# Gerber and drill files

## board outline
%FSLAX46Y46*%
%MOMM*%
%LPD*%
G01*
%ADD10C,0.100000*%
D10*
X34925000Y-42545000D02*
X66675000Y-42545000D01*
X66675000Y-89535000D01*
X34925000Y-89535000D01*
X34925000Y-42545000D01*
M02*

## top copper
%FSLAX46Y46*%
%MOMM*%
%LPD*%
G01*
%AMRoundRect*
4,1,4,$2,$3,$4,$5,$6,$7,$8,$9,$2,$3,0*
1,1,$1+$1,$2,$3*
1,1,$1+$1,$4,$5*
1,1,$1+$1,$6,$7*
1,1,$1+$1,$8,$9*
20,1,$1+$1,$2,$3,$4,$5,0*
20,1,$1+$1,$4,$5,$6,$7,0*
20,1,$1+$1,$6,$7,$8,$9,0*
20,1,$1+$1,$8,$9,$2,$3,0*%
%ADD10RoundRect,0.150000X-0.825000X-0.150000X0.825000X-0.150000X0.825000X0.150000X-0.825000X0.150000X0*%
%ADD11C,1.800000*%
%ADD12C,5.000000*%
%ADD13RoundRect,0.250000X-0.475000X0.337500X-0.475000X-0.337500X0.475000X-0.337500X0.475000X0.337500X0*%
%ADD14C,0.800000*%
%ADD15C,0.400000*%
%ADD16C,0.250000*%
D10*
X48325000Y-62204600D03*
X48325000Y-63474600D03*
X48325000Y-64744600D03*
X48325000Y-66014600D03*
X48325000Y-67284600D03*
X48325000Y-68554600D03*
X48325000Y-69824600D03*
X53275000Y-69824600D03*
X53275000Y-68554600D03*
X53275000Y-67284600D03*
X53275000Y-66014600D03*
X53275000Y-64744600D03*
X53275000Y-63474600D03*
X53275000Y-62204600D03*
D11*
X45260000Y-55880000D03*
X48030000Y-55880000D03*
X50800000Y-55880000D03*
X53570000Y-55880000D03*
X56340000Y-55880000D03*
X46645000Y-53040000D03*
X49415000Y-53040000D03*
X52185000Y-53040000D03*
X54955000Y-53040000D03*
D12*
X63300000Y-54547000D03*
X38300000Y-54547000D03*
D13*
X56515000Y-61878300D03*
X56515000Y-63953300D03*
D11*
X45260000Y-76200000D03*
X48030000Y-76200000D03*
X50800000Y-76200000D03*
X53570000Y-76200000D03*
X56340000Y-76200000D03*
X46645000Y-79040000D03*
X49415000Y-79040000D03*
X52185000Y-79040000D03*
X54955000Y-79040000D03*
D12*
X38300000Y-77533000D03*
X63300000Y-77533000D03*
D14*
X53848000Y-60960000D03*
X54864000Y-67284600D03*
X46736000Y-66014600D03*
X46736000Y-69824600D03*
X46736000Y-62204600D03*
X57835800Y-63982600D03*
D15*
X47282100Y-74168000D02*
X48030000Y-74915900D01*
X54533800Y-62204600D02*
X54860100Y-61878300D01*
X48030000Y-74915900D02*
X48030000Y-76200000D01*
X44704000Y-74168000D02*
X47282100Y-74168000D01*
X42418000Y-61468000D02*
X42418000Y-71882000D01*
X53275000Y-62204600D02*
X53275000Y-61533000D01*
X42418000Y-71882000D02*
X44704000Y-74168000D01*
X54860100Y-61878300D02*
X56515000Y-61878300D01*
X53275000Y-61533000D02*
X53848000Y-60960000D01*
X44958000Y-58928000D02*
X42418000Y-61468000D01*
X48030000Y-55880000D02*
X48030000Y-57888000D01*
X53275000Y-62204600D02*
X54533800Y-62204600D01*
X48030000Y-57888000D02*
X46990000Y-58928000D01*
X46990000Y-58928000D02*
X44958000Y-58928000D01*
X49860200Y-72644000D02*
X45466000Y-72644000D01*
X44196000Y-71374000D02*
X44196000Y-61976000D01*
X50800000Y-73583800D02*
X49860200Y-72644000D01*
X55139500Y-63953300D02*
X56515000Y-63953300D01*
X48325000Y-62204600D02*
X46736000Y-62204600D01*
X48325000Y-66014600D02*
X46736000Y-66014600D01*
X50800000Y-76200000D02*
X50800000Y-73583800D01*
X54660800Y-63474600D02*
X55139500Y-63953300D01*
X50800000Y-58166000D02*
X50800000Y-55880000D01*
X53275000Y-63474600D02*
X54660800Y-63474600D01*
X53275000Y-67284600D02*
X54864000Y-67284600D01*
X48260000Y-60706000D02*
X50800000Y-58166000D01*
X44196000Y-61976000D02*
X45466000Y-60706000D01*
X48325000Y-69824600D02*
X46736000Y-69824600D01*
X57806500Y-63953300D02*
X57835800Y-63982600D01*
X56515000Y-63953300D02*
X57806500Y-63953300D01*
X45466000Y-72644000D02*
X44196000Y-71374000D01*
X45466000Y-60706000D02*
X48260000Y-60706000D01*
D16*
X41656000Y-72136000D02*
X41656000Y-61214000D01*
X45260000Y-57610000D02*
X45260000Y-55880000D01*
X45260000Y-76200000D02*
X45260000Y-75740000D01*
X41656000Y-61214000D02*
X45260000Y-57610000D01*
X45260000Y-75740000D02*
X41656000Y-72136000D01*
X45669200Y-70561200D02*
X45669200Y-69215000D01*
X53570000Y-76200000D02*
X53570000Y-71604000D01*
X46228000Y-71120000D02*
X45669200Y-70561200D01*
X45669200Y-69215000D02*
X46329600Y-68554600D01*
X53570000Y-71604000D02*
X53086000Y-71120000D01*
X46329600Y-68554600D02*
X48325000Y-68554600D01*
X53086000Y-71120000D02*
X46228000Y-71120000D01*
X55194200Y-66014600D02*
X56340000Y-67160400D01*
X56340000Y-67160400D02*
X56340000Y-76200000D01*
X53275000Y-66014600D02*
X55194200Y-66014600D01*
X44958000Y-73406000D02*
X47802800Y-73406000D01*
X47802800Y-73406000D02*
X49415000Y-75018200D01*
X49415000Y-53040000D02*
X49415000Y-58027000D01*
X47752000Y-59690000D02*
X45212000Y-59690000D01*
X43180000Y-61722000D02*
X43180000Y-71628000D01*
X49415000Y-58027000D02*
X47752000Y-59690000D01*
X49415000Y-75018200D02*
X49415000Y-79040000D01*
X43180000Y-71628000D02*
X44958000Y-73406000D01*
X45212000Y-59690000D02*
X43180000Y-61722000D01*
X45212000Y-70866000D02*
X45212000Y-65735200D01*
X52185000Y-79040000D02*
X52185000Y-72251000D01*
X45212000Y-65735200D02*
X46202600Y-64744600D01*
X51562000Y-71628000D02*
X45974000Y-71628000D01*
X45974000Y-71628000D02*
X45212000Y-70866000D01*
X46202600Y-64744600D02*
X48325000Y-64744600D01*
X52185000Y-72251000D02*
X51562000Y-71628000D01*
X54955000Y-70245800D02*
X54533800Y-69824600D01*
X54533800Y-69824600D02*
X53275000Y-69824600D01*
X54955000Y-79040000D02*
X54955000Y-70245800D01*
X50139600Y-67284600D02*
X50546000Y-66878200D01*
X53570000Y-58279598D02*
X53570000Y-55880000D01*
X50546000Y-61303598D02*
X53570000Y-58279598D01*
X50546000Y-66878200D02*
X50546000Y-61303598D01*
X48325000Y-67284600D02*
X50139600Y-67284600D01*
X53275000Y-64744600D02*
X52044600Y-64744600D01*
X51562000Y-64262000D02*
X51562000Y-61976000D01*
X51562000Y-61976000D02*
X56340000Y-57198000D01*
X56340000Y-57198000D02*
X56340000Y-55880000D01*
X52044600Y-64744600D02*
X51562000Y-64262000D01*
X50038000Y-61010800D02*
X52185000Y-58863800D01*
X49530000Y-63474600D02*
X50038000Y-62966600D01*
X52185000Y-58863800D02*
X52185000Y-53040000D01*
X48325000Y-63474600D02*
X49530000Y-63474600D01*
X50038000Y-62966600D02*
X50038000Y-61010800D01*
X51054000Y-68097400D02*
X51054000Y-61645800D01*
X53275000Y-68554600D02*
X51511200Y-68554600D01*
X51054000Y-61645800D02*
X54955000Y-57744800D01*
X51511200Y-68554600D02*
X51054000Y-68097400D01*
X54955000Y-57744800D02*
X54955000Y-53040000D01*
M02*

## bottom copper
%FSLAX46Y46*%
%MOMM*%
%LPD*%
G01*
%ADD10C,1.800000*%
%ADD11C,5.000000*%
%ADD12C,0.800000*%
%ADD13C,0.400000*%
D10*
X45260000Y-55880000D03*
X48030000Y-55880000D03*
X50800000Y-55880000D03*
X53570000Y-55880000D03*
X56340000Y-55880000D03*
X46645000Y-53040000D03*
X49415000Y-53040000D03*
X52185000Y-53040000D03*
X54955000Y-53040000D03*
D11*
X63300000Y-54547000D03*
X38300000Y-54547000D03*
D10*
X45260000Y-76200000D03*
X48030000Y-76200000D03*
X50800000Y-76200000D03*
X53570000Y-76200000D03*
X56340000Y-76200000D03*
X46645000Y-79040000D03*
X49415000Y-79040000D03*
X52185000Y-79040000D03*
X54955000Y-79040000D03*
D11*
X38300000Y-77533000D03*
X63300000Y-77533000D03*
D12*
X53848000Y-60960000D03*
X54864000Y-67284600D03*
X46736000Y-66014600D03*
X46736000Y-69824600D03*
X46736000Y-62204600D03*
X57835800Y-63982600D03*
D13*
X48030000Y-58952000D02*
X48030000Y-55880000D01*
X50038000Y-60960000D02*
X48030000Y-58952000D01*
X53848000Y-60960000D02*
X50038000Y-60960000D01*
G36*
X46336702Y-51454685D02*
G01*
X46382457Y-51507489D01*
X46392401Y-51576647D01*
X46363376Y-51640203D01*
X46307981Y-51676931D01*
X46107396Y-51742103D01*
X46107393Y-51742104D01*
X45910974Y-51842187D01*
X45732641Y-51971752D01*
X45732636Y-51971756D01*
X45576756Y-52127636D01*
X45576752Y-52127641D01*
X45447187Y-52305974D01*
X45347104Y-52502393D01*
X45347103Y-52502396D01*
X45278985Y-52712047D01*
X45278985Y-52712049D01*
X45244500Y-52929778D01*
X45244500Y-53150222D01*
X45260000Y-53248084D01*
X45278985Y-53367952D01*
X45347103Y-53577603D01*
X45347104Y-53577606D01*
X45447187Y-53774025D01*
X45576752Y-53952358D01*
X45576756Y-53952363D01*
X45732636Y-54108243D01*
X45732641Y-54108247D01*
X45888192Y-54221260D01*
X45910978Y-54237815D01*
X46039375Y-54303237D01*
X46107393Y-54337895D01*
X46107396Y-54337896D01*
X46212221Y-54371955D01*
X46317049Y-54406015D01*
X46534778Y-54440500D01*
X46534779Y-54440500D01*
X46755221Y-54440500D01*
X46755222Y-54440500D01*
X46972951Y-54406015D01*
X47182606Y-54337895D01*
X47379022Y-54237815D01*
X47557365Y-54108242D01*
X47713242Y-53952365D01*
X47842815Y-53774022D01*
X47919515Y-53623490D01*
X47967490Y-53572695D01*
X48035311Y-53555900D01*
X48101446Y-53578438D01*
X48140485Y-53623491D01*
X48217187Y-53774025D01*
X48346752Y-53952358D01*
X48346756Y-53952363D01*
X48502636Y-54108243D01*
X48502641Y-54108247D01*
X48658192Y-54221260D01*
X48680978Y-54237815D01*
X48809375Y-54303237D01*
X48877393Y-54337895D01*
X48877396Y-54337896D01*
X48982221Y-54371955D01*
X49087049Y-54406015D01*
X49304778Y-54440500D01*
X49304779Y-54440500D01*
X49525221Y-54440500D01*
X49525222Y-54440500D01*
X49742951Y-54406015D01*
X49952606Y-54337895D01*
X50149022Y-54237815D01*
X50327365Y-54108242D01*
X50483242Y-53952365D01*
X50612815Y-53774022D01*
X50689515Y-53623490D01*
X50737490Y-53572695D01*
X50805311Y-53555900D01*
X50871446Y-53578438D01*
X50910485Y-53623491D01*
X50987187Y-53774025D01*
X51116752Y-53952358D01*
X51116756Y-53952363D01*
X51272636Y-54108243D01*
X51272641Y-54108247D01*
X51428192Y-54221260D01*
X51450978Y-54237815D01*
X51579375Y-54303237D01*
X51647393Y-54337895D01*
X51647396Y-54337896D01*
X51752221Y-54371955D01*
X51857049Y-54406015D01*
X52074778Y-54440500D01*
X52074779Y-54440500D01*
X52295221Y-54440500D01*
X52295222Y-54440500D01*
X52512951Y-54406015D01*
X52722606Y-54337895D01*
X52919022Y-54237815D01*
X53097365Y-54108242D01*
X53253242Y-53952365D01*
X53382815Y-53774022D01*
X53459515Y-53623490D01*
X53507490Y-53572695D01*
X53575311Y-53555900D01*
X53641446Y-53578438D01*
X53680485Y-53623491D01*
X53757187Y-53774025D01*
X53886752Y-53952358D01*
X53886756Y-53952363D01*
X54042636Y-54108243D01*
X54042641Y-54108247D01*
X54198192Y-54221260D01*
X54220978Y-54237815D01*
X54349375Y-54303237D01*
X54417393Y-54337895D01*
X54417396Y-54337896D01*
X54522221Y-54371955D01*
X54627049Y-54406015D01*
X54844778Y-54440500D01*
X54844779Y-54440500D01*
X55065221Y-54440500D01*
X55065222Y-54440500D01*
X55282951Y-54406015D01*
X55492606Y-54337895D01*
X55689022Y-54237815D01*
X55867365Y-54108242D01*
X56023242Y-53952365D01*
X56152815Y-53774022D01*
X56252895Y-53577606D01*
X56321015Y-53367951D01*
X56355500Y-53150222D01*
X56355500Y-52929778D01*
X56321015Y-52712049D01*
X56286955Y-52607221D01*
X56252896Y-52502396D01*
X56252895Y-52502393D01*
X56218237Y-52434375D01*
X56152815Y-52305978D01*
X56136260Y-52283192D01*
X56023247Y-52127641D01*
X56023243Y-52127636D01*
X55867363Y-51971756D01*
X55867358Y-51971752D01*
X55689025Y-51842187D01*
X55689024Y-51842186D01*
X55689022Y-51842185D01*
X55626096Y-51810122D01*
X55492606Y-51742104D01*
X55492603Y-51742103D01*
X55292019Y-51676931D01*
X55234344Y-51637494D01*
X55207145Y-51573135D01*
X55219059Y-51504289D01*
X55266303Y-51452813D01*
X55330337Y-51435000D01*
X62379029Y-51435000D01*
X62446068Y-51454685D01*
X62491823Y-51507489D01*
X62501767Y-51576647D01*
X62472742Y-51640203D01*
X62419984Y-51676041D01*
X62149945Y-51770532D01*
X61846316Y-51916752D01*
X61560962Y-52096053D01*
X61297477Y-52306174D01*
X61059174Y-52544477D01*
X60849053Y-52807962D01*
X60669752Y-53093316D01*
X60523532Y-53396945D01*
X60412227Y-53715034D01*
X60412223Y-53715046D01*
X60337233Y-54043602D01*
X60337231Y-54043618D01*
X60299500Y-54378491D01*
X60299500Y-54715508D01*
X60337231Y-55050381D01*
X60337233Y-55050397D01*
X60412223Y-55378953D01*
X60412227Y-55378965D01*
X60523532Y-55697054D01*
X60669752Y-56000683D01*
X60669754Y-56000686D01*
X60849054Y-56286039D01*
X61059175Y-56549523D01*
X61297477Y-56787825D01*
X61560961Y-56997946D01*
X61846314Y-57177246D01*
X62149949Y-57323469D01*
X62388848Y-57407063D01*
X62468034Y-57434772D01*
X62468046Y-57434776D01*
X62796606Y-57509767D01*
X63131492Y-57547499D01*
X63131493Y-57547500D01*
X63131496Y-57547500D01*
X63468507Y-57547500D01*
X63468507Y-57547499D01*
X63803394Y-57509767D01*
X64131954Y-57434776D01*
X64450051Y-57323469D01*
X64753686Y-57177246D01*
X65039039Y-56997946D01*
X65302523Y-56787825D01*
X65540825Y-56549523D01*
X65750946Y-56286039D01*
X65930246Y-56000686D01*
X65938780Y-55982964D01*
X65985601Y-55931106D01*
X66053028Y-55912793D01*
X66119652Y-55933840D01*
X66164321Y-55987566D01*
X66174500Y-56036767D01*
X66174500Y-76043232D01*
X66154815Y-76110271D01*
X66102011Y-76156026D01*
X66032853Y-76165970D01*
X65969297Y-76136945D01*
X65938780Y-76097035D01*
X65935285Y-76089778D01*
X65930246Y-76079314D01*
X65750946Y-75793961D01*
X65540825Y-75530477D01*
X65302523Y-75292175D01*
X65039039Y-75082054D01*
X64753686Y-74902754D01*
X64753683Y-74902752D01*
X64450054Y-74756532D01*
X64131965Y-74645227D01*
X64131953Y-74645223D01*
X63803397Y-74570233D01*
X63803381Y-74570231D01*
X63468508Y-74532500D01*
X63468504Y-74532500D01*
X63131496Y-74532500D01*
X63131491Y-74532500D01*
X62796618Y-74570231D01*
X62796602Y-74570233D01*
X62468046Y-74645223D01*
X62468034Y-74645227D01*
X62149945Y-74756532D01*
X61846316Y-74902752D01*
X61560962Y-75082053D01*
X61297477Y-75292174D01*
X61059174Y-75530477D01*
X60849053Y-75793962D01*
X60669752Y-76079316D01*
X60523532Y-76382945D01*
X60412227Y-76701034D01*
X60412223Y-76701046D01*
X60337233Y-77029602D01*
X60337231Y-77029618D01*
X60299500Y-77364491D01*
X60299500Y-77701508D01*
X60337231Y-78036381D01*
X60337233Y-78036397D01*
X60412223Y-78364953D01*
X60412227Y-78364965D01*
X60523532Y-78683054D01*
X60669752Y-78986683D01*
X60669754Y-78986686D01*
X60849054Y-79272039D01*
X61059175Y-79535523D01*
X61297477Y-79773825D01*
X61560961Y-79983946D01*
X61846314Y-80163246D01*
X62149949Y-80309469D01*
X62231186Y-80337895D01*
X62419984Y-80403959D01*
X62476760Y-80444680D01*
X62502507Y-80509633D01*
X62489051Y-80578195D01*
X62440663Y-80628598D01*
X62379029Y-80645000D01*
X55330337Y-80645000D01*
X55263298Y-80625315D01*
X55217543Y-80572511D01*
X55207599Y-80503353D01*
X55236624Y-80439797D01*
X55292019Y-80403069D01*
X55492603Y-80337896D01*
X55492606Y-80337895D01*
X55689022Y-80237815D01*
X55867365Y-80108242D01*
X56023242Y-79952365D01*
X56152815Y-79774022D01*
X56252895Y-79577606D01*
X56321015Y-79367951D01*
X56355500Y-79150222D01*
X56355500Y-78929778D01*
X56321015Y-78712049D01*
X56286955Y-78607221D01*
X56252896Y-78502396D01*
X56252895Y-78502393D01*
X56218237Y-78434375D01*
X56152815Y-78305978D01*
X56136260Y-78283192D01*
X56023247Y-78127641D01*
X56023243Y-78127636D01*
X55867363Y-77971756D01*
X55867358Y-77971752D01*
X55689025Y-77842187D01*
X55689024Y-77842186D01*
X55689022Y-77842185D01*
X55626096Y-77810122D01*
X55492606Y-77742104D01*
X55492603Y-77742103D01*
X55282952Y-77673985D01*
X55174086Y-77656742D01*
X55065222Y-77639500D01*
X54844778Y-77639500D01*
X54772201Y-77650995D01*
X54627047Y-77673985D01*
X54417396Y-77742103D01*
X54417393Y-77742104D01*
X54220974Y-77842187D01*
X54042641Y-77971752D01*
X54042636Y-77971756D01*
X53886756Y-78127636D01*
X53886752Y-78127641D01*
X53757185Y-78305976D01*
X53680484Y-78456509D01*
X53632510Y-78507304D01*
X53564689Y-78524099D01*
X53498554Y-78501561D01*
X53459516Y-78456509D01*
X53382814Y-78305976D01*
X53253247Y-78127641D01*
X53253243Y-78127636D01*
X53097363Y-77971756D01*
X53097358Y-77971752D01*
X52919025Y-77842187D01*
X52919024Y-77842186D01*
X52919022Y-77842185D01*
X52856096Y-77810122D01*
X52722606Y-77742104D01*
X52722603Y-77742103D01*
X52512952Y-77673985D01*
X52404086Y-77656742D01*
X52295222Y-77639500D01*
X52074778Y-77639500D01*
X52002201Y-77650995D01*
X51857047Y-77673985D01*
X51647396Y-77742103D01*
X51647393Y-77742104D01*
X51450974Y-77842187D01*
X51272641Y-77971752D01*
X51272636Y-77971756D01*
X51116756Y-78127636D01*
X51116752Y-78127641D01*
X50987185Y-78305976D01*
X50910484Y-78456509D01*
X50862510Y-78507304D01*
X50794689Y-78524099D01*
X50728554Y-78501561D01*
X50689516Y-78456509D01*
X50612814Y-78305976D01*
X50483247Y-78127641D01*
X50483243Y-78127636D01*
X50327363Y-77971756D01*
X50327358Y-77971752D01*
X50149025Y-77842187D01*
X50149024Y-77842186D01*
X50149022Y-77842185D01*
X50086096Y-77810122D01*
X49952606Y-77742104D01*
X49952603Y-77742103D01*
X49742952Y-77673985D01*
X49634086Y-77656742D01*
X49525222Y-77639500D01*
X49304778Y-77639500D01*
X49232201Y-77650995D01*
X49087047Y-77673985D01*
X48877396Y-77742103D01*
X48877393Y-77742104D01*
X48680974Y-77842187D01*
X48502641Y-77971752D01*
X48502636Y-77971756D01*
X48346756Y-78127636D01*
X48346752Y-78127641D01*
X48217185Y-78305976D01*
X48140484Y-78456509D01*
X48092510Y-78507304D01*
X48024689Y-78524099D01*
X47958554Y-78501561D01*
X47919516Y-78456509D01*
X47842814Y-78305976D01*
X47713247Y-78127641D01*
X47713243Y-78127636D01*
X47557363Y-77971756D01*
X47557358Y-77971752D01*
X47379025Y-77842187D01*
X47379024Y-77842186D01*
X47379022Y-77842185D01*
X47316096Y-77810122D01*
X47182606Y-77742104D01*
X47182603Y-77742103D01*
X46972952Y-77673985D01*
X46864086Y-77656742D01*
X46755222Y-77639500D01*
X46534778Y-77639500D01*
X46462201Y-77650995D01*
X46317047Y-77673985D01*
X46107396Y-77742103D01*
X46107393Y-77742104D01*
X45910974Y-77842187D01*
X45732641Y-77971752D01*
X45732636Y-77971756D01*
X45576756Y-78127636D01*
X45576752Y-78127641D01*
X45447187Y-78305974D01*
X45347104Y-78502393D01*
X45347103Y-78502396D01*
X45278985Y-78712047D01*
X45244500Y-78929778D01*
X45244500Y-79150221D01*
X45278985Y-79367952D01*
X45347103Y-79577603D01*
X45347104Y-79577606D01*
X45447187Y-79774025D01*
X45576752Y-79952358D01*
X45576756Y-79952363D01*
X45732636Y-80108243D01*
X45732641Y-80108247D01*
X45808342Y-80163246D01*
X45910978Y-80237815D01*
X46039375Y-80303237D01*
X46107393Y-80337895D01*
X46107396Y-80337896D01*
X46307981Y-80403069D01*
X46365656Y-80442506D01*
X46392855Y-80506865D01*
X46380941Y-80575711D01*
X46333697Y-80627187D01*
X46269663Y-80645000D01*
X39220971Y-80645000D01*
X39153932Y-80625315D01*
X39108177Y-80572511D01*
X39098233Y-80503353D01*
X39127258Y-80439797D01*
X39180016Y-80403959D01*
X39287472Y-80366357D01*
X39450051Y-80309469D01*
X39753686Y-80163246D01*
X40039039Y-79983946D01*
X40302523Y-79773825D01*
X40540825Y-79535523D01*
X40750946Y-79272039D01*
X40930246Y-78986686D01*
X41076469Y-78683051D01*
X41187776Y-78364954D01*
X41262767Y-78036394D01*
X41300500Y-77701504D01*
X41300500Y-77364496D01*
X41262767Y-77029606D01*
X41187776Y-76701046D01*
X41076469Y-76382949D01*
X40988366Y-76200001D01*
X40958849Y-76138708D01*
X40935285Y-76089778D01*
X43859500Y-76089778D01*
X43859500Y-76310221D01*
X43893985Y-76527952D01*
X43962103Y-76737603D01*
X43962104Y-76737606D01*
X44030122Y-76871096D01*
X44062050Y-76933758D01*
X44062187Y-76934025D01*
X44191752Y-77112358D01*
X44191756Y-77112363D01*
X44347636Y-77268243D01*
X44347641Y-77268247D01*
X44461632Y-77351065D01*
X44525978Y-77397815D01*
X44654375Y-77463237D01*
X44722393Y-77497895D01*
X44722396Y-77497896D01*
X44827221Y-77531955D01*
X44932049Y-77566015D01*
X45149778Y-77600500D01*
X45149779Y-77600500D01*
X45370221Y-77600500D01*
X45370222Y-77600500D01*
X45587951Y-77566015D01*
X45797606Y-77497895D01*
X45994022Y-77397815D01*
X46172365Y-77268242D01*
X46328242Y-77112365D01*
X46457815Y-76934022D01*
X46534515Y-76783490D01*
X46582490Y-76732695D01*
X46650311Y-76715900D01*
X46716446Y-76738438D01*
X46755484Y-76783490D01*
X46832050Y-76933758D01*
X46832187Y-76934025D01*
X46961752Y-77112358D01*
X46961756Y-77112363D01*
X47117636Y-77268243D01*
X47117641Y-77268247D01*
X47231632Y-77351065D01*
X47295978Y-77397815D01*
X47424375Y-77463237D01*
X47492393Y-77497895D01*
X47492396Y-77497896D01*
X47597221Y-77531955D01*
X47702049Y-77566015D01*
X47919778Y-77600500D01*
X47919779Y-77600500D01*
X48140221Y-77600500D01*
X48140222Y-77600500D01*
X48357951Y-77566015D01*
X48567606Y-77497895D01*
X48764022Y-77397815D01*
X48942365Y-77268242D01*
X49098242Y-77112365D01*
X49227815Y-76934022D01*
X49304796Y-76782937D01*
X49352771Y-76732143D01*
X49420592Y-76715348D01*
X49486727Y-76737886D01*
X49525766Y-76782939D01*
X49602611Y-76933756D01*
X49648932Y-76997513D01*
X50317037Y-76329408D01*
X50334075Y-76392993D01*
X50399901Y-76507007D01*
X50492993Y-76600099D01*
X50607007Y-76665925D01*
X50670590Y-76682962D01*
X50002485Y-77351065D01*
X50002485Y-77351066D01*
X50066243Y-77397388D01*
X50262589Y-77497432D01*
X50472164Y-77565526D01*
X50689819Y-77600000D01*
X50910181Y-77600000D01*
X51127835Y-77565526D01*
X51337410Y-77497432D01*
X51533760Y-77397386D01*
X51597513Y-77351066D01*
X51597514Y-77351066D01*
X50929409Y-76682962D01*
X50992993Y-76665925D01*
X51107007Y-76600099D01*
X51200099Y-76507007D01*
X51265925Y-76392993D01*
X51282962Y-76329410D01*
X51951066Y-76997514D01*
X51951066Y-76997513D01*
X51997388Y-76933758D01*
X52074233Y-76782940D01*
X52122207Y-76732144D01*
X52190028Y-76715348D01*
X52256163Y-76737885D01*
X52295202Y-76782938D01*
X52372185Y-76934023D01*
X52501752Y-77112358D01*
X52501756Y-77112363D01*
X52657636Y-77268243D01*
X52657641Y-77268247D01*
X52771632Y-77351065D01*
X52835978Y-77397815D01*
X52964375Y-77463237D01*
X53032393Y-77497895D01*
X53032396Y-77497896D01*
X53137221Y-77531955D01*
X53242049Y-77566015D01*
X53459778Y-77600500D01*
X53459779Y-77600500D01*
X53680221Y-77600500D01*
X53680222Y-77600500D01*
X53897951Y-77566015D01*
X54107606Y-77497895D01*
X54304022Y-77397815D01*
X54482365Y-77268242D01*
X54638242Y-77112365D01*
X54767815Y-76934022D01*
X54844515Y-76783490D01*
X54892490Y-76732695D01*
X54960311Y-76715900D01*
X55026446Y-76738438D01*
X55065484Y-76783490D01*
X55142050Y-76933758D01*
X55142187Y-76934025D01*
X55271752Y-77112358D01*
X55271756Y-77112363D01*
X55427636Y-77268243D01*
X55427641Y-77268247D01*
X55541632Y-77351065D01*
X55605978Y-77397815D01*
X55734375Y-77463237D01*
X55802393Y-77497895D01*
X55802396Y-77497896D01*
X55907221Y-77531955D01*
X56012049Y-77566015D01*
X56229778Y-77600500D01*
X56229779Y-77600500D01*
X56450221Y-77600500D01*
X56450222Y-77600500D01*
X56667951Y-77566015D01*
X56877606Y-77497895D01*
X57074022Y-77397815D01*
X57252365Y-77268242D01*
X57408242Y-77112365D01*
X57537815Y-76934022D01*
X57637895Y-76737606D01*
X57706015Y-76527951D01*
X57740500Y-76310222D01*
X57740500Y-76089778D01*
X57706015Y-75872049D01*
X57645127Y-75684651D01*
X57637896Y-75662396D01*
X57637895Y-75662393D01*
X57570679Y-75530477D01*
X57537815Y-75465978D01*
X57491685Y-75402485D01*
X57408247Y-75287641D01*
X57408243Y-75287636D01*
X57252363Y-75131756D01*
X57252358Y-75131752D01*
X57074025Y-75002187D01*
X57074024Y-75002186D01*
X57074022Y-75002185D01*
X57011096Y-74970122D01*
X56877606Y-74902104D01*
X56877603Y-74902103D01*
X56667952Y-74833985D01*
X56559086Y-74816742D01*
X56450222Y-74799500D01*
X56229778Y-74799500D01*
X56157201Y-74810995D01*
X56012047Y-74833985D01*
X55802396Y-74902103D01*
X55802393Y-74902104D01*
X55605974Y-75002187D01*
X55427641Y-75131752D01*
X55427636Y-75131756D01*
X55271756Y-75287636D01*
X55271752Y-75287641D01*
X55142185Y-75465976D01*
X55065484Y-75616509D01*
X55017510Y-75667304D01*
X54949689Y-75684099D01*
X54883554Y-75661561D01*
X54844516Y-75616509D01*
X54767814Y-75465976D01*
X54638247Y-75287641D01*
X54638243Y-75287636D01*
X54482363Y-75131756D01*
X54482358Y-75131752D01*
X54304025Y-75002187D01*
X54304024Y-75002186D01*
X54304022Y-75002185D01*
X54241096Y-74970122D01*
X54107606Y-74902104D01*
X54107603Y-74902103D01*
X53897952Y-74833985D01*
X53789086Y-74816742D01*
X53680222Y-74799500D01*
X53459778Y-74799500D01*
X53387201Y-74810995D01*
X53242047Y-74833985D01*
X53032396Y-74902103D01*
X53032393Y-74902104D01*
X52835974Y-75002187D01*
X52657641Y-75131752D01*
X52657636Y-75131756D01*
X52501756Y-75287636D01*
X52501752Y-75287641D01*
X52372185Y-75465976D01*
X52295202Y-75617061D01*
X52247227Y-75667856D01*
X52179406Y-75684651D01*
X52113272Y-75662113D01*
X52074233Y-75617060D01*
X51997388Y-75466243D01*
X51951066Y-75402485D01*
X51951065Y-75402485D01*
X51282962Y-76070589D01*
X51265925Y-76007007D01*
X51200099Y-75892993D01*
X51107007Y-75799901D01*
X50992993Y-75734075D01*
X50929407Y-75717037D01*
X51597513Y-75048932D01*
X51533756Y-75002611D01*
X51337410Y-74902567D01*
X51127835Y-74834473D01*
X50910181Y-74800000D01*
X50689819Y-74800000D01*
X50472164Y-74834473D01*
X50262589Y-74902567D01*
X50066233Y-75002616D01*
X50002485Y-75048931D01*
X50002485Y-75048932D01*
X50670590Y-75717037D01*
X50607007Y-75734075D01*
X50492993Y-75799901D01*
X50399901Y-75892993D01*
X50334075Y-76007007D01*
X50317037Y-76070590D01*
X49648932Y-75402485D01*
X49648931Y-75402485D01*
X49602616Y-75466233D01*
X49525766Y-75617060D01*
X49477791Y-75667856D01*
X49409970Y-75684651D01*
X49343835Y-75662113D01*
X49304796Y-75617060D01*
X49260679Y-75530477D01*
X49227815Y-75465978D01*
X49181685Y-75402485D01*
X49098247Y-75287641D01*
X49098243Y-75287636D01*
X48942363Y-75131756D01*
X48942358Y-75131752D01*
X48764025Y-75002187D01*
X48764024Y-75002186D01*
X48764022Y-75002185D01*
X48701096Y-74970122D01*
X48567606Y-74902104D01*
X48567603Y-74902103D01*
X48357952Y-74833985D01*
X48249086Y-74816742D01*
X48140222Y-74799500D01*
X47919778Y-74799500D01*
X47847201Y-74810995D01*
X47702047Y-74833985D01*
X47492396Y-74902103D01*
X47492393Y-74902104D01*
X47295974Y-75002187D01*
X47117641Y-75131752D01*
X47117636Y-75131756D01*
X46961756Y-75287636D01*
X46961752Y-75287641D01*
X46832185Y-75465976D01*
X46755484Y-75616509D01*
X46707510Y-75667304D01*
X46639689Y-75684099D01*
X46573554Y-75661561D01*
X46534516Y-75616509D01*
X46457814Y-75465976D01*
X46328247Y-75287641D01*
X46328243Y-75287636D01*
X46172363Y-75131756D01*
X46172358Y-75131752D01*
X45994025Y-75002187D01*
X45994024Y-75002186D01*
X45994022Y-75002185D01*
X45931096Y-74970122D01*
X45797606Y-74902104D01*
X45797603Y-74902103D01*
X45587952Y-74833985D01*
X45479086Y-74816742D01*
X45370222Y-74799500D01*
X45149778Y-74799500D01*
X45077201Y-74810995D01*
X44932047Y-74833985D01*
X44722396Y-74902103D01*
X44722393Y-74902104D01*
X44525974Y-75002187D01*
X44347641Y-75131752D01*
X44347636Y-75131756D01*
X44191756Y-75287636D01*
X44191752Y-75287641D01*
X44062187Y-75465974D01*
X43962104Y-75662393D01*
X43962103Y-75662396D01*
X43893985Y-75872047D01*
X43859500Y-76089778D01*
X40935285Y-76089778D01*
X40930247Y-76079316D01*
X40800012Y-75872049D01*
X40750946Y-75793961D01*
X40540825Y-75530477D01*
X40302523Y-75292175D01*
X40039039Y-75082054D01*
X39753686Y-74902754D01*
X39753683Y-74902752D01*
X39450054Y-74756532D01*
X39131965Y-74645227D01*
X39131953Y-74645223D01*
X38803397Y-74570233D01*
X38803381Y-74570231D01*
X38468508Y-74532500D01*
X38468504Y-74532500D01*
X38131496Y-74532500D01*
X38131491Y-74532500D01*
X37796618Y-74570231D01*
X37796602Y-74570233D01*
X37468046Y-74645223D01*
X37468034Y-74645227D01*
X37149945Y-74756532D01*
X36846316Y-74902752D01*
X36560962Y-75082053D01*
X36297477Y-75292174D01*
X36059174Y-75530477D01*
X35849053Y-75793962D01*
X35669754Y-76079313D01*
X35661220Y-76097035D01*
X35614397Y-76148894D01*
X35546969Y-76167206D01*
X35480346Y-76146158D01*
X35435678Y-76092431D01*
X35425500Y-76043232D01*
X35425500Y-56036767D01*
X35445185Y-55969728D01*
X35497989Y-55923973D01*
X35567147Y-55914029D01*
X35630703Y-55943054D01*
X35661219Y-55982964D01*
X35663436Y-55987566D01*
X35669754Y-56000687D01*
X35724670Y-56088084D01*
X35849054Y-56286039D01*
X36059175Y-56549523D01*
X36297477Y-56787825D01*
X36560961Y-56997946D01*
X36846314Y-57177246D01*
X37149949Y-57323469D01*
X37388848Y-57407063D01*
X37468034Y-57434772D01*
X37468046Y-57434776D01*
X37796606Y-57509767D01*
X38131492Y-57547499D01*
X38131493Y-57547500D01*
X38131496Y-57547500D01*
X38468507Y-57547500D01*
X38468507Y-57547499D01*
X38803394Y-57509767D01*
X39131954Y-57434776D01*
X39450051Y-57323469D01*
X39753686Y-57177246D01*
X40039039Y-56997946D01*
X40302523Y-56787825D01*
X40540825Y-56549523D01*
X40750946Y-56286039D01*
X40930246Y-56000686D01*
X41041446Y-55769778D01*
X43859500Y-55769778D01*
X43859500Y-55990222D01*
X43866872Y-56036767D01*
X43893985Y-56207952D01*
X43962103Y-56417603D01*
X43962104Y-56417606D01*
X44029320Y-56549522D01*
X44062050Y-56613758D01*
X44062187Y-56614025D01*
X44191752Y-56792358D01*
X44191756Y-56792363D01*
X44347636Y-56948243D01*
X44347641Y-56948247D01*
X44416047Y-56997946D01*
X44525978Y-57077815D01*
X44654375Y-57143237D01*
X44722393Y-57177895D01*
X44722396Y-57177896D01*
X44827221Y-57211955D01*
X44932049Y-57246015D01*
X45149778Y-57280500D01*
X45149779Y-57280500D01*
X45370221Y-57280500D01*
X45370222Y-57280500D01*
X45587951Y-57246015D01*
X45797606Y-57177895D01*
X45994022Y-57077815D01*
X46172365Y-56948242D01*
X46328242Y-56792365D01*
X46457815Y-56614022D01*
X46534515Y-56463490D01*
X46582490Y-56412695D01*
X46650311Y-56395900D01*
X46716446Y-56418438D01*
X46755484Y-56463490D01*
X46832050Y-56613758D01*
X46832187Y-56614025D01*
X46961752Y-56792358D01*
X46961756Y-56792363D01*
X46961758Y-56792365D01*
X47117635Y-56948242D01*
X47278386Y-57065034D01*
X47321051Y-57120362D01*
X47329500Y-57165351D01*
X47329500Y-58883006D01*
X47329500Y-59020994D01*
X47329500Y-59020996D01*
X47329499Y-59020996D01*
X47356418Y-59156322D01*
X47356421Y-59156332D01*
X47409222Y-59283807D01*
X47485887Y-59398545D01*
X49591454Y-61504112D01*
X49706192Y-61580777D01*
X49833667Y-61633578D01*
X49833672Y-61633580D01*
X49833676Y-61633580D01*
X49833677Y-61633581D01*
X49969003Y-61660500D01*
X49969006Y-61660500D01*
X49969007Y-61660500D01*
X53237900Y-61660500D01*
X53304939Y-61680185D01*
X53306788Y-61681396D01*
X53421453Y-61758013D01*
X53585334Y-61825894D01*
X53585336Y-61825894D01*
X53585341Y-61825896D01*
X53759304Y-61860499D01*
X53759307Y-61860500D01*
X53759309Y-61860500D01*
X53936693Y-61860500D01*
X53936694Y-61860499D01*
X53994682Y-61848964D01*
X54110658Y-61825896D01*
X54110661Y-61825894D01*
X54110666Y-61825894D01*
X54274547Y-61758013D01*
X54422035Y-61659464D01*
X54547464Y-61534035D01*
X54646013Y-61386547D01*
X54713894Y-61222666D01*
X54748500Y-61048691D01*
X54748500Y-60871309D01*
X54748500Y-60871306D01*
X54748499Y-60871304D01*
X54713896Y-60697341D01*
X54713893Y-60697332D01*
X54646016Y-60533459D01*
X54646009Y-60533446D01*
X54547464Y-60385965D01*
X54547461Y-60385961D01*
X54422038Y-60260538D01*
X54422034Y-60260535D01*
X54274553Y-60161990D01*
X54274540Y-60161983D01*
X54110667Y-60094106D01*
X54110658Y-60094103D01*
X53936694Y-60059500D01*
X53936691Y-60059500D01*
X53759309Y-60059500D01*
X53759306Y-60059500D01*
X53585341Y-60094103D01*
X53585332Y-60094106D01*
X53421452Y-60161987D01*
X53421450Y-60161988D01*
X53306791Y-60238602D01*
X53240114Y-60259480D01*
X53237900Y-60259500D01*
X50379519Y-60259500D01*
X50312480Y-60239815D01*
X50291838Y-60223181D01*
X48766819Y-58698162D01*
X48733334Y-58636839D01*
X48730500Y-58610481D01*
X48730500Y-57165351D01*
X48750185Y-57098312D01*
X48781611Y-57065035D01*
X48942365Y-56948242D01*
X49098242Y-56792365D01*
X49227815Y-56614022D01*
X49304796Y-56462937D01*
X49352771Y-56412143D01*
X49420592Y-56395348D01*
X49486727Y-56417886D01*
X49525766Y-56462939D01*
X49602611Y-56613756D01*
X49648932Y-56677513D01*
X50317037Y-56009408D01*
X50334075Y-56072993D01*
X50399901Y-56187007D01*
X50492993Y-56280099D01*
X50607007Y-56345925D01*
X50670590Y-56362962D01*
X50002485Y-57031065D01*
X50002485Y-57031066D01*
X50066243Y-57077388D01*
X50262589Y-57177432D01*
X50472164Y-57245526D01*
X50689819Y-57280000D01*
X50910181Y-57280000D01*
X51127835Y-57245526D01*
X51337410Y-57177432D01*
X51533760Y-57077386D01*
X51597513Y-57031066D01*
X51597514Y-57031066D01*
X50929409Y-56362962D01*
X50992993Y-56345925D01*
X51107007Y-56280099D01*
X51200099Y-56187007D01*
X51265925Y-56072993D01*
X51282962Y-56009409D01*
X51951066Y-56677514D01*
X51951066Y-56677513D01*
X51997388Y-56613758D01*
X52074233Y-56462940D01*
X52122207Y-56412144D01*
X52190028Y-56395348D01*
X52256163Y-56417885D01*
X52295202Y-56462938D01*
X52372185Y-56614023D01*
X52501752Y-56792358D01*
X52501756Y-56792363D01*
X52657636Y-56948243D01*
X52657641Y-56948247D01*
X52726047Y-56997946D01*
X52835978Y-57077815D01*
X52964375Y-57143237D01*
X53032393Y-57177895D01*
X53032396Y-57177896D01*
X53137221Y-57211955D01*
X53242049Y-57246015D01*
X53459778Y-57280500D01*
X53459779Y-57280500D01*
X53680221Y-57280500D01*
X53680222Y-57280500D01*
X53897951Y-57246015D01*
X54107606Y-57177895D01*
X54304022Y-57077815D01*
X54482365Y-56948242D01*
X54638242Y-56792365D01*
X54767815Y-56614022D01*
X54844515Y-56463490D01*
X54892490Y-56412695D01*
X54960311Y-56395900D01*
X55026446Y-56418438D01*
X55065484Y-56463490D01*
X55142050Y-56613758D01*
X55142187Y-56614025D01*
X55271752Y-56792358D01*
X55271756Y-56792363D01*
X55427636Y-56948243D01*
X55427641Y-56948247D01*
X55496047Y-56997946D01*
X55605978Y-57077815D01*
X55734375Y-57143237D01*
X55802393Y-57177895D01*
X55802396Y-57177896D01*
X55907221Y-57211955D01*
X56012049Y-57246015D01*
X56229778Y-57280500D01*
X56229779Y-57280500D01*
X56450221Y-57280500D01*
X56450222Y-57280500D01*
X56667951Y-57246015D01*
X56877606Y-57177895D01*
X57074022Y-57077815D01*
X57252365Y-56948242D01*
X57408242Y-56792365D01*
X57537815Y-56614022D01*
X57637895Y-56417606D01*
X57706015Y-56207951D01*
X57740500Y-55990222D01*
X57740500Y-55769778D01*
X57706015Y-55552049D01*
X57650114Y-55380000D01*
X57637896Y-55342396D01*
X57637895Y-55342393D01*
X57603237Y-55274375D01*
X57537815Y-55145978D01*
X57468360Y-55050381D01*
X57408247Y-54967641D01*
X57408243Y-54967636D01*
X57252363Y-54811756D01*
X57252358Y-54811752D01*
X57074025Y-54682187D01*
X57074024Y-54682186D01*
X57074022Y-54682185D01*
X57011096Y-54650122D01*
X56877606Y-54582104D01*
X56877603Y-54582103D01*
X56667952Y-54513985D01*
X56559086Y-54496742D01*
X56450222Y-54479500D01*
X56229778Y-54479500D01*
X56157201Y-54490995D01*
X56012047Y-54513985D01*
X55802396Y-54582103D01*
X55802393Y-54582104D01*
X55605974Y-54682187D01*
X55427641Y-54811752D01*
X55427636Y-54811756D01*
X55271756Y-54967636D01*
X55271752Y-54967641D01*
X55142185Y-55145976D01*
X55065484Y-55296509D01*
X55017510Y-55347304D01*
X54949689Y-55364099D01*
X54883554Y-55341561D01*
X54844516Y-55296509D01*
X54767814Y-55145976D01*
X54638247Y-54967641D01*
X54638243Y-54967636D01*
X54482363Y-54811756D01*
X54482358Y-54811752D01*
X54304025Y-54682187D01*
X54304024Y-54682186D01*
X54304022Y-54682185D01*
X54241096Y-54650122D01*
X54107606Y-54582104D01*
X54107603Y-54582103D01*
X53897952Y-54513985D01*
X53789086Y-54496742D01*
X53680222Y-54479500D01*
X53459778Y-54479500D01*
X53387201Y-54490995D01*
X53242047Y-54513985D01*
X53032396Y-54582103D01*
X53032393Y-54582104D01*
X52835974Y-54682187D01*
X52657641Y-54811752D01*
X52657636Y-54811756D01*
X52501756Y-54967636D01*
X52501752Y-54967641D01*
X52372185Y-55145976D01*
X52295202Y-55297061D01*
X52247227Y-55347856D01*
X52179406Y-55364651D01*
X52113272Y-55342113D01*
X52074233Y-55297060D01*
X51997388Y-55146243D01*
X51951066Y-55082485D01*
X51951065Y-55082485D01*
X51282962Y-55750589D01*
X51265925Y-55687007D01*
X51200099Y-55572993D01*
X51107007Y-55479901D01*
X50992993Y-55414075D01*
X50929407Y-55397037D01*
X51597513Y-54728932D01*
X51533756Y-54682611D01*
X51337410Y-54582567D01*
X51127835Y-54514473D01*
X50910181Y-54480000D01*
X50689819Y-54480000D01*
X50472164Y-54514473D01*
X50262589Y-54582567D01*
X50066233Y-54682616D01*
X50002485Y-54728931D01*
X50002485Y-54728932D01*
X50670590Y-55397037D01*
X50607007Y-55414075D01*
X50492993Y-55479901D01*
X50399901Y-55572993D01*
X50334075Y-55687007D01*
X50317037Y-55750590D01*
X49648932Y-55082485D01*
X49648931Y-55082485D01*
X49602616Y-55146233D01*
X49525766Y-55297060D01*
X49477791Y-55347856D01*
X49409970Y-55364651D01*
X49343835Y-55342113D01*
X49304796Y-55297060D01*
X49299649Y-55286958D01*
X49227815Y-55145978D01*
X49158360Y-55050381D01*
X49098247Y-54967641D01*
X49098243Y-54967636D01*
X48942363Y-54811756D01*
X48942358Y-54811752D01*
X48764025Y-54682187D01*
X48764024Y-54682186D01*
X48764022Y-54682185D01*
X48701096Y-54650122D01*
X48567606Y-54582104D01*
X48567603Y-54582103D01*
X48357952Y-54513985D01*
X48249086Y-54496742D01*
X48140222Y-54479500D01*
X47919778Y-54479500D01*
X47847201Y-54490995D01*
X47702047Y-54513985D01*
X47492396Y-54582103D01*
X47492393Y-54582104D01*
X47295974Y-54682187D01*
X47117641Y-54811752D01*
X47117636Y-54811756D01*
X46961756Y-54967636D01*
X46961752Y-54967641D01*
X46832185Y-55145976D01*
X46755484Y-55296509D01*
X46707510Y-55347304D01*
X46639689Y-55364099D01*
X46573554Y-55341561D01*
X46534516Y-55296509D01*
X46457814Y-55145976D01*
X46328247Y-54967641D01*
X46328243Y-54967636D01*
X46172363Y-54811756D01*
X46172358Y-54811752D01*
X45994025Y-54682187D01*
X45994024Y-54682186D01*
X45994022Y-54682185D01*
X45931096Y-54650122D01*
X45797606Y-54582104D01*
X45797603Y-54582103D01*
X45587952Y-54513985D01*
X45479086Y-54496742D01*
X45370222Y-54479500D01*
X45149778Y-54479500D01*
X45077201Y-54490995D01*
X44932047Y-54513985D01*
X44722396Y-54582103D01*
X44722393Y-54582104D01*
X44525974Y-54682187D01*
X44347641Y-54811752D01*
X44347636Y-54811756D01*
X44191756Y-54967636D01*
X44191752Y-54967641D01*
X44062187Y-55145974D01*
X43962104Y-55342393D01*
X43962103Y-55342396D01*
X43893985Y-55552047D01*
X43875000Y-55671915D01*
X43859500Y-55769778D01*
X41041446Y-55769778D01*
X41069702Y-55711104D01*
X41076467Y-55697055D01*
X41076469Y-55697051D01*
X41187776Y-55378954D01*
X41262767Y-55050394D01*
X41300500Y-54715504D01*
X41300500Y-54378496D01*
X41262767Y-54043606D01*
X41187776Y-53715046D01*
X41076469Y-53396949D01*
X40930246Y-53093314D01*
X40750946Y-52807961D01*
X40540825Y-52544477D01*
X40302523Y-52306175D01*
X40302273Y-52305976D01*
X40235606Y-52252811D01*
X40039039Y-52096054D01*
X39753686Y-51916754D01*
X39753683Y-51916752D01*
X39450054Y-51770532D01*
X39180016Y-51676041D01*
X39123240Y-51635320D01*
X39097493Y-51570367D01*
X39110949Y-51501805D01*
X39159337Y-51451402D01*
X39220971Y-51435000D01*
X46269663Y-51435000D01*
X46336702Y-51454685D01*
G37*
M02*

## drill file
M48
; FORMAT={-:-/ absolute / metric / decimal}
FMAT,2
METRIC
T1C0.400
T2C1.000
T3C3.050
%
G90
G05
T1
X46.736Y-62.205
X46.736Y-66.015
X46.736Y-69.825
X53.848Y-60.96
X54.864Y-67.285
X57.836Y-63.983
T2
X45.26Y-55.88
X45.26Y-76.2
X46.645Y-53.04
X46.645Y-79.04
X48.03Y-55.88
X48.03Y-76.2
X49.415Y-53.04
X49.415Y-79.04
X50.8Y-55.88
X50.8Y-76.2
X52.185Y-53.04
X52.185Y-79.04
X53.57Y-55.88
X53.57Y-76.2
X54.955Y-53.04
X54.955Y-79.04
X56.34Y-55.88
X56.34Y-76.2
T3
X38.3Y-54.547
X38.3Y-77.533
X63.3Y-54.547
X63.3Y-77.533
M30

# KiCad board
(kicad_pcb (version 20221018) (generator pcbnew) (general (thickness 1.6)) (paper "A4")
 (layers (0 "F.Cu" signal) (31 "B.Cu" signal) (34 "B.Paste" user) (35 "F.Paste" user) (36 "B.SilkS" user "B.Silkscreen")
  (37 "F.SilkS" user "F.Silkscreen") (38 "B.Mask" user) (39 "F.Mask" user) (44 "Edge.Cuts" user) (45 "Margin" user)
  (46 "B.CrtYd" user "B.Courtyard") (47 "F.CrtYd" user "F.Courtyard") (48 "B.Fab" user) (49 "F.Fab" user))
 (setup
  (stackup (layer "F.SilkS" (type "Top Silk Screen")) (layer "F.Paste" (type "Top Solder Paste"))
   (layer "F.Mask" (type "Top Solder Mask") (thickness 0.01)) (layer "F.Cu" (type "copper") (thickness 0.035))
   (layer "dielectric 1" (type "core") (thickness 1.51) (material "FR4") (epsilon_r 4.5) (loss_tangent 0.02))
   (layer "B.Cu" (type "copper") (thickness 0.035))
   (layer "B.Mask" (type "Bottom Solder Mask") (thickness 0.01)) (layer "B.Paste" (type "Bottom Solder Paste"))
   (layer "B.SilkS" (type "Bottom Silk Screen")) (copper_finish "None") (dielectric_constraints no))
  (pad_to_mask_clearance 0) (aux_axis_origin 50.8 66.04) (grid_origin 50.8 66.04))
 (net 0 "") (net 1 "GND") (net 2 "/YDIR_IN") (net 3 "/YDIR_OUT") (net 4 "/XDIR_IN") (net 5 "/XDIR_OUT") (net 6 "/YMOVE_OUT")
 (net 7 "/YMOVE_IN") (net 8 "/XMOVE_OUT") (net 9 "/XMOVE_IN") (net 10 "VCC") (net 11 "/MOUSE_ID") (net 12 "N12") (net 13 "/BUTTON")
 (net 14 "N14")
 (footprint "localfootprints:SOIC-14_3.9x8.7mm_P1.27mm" (layer "F.Cu") (at 50.8 66.0146)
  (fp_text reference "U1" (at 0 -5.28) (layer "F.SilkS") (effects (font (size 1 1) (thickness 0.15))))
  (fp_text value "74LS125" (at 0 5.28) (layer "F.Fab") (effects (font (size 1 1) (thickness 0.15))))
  (pad "1" smd roundrect (at -2.475 -3.81) (size 1.95 0.6) (layers "F.Cu" "F.Paste" "F.Mask") (roundrect_rratio 0.25) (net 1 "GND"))
  (pad "2" smd roundrect (at -2.475 -2.54) (size 1.95 0.6) (layers "F.Cu" "F.Paste" "F.Mask") (roundrect_rratio 0.25) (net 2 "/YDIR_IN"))
  (pad "3" smd roundrect (at -2.475 -1.27) (size 1.95 0.6) (layers "F.Cu" "F.Paste" "F.Mask") (roundrect_rratio 0.25) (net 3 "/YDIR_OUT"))
  (pad "4" smd roundrect (at -2.475 0) (size 1.95 0.6) (layers "F.Cu" "F.Paste" "F.Mask") (roundrect_rratio 0.25) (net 1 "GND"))
  (pad "5" smd roundrect (at -2.475 1.27) (size 1.95 0.6) (layers "F.Cu" "F.Paste" "F.Mask") (roundrect_rratio 0.25) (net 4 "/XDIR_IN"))
  (pad "6" smd roundrect (at -2.475 2.54) (size 1.95 0.6) (layers "F.Cu" "F.Paste" "F.Mask") (roundrect_rratio 0.25) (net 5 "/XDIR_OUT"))
  (pad "7" smd roundrect (at -2.475 3.81) (size 1.95 0.6) (layers "F.Cu" "F.Paste" "F.Mask") (roundrect_rratio 0.25) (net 1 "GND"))
  (pad "8" smd roundrect (at 2.475 3.81) (size 1.95 0.6) (layers "F.Cu" "F.Paste" "F.Mask") (roundrect_rratio 0.25) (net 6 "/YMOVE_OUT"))
  (pad "9" smd roundrect (at 2.475 2.54) (size 1.95 0.6) (layers "F.Cu" "F.Paste" "F.Mask") (roundrect_rratio 0.25) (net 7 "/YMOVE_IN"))
  (pad "10" smd roundrect (at 2.475 1.27) (size 1.95 0.6) (layers "F.Cu" "F.Paste" "F.Mask") (roundrect_rratio 0.25) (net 1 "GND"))
  (pad "11" smd roundrect (at 2.475 0) (size 1.95 0.6) (layers "F.Cu" "F.Paste" "F.Mask") (roundrect_rratio 0.25) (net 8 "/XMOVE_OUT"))
  (pad "12" smd roundrect (at 2.475 -1.27) (size 1.95 0.6) (layers "F.Cu" "F.Paste" "F.Mask") (roundrect_rratio 0.25) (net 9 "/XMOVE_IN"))
  (pad "13" smd roundrect (at 2.475 -2.54) (size 1.95 0.6) (layers "F.Cu" "F.Paste" "F.Mask") (roundrect_rratio 0.25) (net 1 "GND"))
  (pad "14" smd roundrect (at 2.475 -3.81) (size 1.95 0.6) (layers "F.Cu" "F.Paste" "F.Mask") (roundrect_rratio 0.25) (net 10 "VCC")))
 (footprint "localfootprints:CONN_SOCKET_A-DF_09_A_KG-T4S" (layer "F.Cu") (at 50.8 55.88)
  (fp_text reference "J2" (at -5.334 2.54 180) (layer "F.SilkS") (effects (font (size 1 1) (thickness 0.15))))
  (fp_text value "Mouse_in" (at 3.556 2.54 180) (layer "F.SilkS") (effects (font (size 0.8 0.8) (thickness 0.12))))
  (pad "1" thru_hole circle (at -5.54 0 180) (size 1.8 1.8) (drill 1) (layers "*.Cu" "*.Mask") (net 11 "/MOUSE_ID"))
  (pad "2" thru_hole circle (at -2.77 0 180) (size 1.8 1.8) (drill 1) (layers "*.Cu" "*.Mask") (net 10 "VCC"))
  (pad "3" thru_hole circle (at 0 0 180) (size 1.8 1.8) (drill 1) (layers "*.Cu" "*.Mask") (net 1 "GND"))
  (pad "4" thru_hole circle (at 2.77 0 180) (size 1.8 1.8) (drill 1) (layers "*.Cu" "*.Mask") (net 4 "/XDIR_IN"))
  (pad "5" thru_hole circle (at 5.54 0 180) (size 1.8 1.8) (drill 1) (layers "*.Cu" "*.Mask") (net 9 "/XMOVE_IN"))
  (pad "6" thru_hole circle (at -4.155 -2.84 180) (size 1.8 1.8) (drill 1) (layers "*.Cu" "*.Mask") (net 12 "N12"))
  (pad "7" thru_hole circle (at -1.385 -2.84 180) (size 1.8 1.8) (drill 1) (layers "*.Cu" "*.Mask") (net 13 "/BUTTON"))
  (pad "8" thru_hole circle (at 1.385 -2.84 180) (size 1.8 1.8) (drill 1) (layers "*.Cu" "*.Mask") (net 2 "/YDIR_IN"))
  (pad "9" thru_hole circle (at 4.155 -2.84 180) (size 1.8 1.8) (drill 1) (layers "*.Cu" "*.Mask") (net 7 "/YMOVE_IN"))
  (pad "10" thru_hole circle (at 12.5 -1.333 180) (size 5 5) (drill 3.05) (layers "*.Cu" "*.Mask"))
  (pad "11" thru_hole circle (at -12.5 -1.333 180) (size 5 5) (drill 3.05) (layers "*.Cu" "*.Mask")))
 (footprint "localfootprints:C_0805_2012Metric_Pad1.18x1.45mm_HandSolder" (layer "F.Cu") (at 56.515 62.9158 -90)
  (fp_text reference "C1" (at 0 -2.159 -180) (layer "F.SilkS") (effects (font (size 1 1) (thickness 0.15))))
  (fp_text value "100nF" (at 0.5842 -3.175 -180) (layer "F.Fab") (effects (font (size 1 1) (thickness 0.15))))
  (pad "1" smd roundrect (at -1.0375 0 270) (size 1.175 1.45) (layers "F.Cu" "F.Paste" "F.Mask") (roundrect_rratio 0.2127659574)
   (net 10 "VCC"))
  (pad "2" smd roundrect (at 1.0375 0 270) (size 1.175 1.45) (layers "F.Cu" "F.Paste" "F.Mask") (roundrect_rratio 0.2127659574)
   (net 1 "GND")))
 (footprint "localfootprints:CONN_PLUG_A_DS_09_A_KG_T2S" (layer "F.Cu") (at 50.8 76.2 180)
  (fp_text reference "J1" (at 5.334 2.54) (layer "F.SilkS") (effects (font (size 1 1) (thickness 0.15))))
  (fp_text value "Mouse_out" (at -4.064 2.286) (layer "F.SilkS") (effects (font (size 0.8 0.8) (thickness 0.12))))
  (pad "1" thru_hole circle (at 5.54 0) (size 1.8 1.8) (drill 1) (layers "*.Cu" "*.Mask") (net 11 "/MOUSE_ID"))
  (pad "2" thru_hole circle (at 2.77 0) (size 1.8 1.8) (drill 1) (layers "*.Cu" "*.Mask") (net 10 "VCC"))
  (pad "3" thru_hole circle (at 0 0) (size 1.8 1.8) (drill 1) (layers "*.Cu" "*.Mask") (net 1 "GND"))
  (pad "4" thru_hole circle (at -2.77 0) (size 1.8 1.8) (drill 1) (layers "*.Cu" "*.Mask") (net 5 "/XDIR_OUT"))
  (pad "5" thru_hole circle (at -5.54 0) (size 1.8 1.8) (drill 1) (layers "*.Cu" "*.Mask") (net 8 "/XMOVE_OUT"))
  (pad "6" thru_hole circle (at 4.155 -2.84) (size 1.8 1.8) (drill 1) (layers "*.Cu" "*.Mask") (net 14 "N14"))
  (pad "7" thru_hole circle (at 1.385 -2.84) (size 1.8 1.8) (drill 1) (layers "*.Cu" "*.Mask") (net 13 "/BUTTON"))
  (pad "8" thru_hole circle (at -1.385 -2.84) (size 1.8 1.8) (drill 1) (layers "*.Cu" "*.Mask") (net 3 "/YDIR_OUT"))
  (pad "9" thru_hole circle (at -4.155 -2.84) (size 1.8 1.8) (drill 1) (layers "*.Cu" "*.Mask") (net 6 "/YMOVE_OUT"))
  (pad "10" thru_hole circle (at 12.5 -1.333) (size 5 5) (drill 3.05) (layers "*.Cu" "*.Mask"))
  (pad "11" thru_hole circle (at -12.5 -1.333) (size 5 5) (drill 3.05) (layers "*.Cu" "*.Mask")))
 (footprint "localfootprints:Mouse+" (layer "B.Cu") (at 50.8 66.04 180)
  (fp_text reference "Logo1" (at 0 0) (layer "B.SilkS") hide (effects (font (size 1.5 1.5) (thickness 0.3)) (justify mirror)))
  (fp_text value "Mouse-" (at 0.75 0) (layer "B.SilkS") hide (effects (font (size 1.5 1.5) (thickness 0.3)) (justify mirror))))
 (gr_rect (start 34.925 42.545) (end 66.675 89.535) (stroke (width 0.1) (type default)) (fill none) (layer "Edge.Cuts"))
 (segment (start 47.2821 74.168) (end 48.03 74.9159) (width 0.4) (layer "F.Cu") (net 10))
 (segment (start 54.5338 62.2046) (end 54.8601 61.8783) (width 0.4) (layer "F.Cu") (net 10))
 (segment (start 48.03 74.9159) (end 48.03 76.2) (width 0.4) (layer "F.Cu") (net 10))
 (segment (start 44.704 74.168) (end 47.2821 74.168) (width 0.4) (layer "F.Cu") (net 10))
 (segment (start 42.418 61.468) (end 42.418 71.882) (width 0.4) (layer "F.Cu") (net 10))
 (segment (start 53.275 62.2046) (end 53.275 61.533) (width 0.4) (layer "F.Cu") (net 10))
 (segment (start 42.418 71.882) (end 44.704 74.168) (width 0.4) (layer "F.Cu") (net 10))
 (segment (start 54.8601 61.8783) (end 56.515 61.8783) (width 0.4) (layer "F.Cu") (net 10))
 (segment (start 53.275 61.533) (end 53.848 60.96) (width 0.4) (layer "F.Cu") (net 10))
 (segment (start 44.958 58.928) (end 42.418 61.468) (width 0.4) (layer "F.Cu") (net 10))
 (segment (start 48.03 55.88) (end 48.03 57.888) (width 0.4) (layer "F.Cu") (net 10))
 (segment (start 53.275 62.2046) (end 54.5338 62.2046) (width 0.4) (layer "F.Cu") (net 10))
 (segment (start 48.03 57.888) (end 46.99 58.928) (width 0.4) (layer "F.Cu") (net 10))
 (segment (start 46.99 58.928) (end 44.958 58.928) (width 0.4) (layer "F.Cu") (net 10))
 (via (at 53.848 60.96) (size 0.8) (drill 0.4) (layers "F.Cu" "B.Cu") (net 10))
 (segment (start 48.03 58.952) (end 48.03 55.88) (width 0.4) (layer "B.Cu") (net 10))
 (segment (start 50.038 60.96) (end 48.03 58.952) (width 0.4) (layer "B.Cu") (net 10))
 (segment (start 53.848 60.96) (end 50.038 60.96) (width 0.4) (layer "B.Cu") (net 10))
 (segment (start 49.8602 72.644) (end 45.466 72.644) (width 0.4) (layer "F.Cu") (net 1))
 (segment (start 44.196 71.374) (end 44.196 61.976) (width 0.4) (layer "F.Cu") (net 1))
 (segment (start 50.8 73.5838) (end 49.8602 72.644) (width 0.4) (layer "F.Cu") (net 1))
 (segment (start 55.1395 63.9533) (end 56.515 63.9533) (width 0.4) (layer "F.Cu") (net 1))
 (segment (start 48.325 62.2046) (end 46.736 62.2046) (width 0.4) (layer "F.Cu") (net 1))
 (segment (start 48.325 66.0146) (end 46.736 66.0146) (width 0.4) (layer "F.Cu") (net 1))
 (segment (start 50.8 76.2) (end 50.8 73.5838) (width 0.4) (layer "F.Cu") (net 1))
 (segment (start 54.6608 63.4746) (end 55.1395 63.9533) (width 0.4) (layer "F.Cu") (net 1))
 (segment (start 50.8 58.166) (end 50.8 55.88) (width 0.4) (layer "F.Cu") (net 1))
 (segment (start 53.275 63.4746) (end 54.6608 63.4746) (width 0.4) (layer "F.Cu") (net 1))
 (segment (start 53.275 67.2846) (end 54.864 67.2846) (width 0.4) (layer "F.Cu") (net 1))
 (segment (start 48.26 60.706) (end 50.8 58.166) (width 0.4) (layer "F.Cu") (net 1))
 (segment (start 44.196 61.976) (end 45.466 60.706) (width 0.4) (layer "F.Cu") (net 1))
 (segment (start 48.325 69.8246) (end 46.736 69.8246) (width 0.4) (layer "F.Cu") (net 1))
 (segment (start 57.8065 63.9533) (end 57.8358 63.9826) (width 0.4) (layer "F.Cu") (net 1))
 (segment (start 56.515 63.9533) (end 57.8065 63.9533) (width 0.4) (layer "F.Cu") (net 1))
 (segment (start 45.466 72.644) (end 44.196 71.374) (width 0.4) (layer "F.Cu") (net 1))
 (segment (start 45.466 60.706) (end 48.26 60.706) (width 0.4) (layer "F.Cu") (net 1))
 (via (at 54.864 67.2846) (size 0.8) (drill 0.4) (layers "F.Cu" "B.Cu") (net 1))
 (via (at 46.736 66.0146) (size 0.8) (drill 0.4) (layers "F.Cu" "B.Cu") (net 1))
 (via (at 46.736 69.8246) (size 0.8) (drill 0.4) (layers "F.Cu" "B.Cu") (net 1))
 (via (at 46.736 62.2046) (size 0.8) (drill 0.4) (layers "F.Cu" "B.Cu") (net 1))
 (via (at 57.8358 63.9826) (size 0.8) (drill 0.4) (layers "F.Cu" "B.Cu") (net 1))
 (segment (start 41.656 72.136) (end 41.656 61.214) (width 0.25) (layer "F.Cu") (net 11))
 (segment (start 45.26 57.61) (end 45.26 55.88) (width 0.25) (layer "F.Cu") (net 11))
 (segment (start 45.26 76.2) (end 45.26 75.74) (width 0.25) (layer "F.Cu") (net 11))
 (segment (start 41.656 61.214) (end 45.26 57.61) (width 0.25) (layer "F.Cu") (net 11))
 (segment (start 45.26 75.74) (end 41.656 72.136) (width 0.25) (layer "F.Cu") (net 11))
 (segment (start 45.6692 70.5612) (end 45.6692 69.215) (width 0.25) (layer "F.Cu") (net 5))
 (segment (start 53.57 76.2) (end 53.57 71.604) (width 0.25) (layer "F.Cu") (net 5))
 (segment (start 46.228 71.12) (end 45.6692 70.5612) (width 0.25) (layer "F.Cu") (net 5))
 (segment (start 45.6692 69.215) (end 46.3296 68.5546) (width 0.25) (layer "F.Cu") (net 5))
 (segment (start 53.57 71.604) (end 53.086 71.12) (width 0.25) (layer "F.Cu") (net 5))
 (segment (start 46.3296 68.5546) (end 48.325 68.5546) (width 0.25) (layer "F.Cu") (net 5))
 (segment (start 53.086 71.12) (end 46.228 71.12) (width 0.25) (layer "F.Cu") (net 5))
 (segment (start 55.1942 66.0146) (end 56.34 67.1604) (width 0.25) (layer "F.Cu") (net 8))
 (segment (start 56.34 67.1604) (end 56.34 76.2) (width 0.25) (layer "F.Cu") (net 8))
 (segment (start 53.275 66.0146) (end 55.1942 66.0146) (width 0.25) (layer "F.Cu") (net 8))
 (segment (start 44.958 73.406) (end 47.8028 73.406) (width 0.25) (layer "F.Cu") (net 13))
 (segment (start 47.8028 73.406) (end 49.415 75.0182) (width 0.25) (layer "F.Cu") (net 13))
 (segment (start 49.415 53.04) (end 49.415 58.027) (width 0.25) (layer "F.Cu") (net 13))
 (segment (start 47.752 59.69) (end 45.212 59.69) (width 0.25) (layer "F.Cu") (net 13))
 (segment (start 43.18 61.722) (end 43.18 71.628) (width 0.25) (layer "F.Cu") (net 13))
 (segment (start 49.415 58.027) (end 47.752 59.69) (width 0.25) (layer "F.Cu") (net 13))
 (segment (start 49.415 75.0182) (end 49.415 79.04) (width 0.25) (layer "F.Cu") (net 13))
 (segment (start 43.18 71.628) (end 44.958 73.406) (width 0.25) (layer "F.Cu") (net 13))
 (segment (start 45.212 59.69) (end 43.18 61.722) (width 0.25) (layer "F.Cu") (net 13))
 (segment (start 45.212 70.866) (end 45.212 65.7352) (width 0.25) (layer "F.Cu") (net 3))
 (segment (start 52.185 79.04) (end 52.185 72.251) (width 0.25) (layer "F.Cu") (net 3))
 (segment (start 45.212 65.7352) (end 46.2026 64.7446) (width 0.25) (layer "F.Cu") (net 3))
 (segment (start 51.562 71.628) (end 45.974 71.628) (width 0.25) (layer "F.Cu") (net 3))
 (segment (start 45.974 71.628) (end 45.212 70.866) (width 0.25) (layer "F.Cu") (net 3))
 (segment (start 46.2026 64.7446) (end 48.325 64.7446) (width 0.25) (layer "F.Cu") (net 3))
 (segment (start 52.185 72.251) (end 51.562 71.628) (width 0.25) (layer "F.Cu") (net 3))
 (segment (start 54.955 70.2458) (end 54.5338 69.8246) (width 0.25) (layer "F.Cu") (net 6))
 (segment (start 54.5338 69.8246) (end 53.275 69.8246) (width 0.25) (layer "F.Cu") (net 6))
 (segment (start 54.955 79.04) (end 54.955 70.2458) (width 0.25) (layer "F.Cu") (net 6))
 (segment (start 50.1396 67.2846) (end 50.546 66.8782) (width 0.25) (layer "F.Cu") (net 4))
 (segment (start 53.57 58.279598) (end 53.57 55.88) (width 0.25) (layer "F.Cu") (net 4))
 (segment (start 50.546 61.303598) (end 53.57 58.279598) (width 0.25) (layer "F.Cu") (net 4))
 (segment (start 50.546 66.8782) (end 50.546 61.303598) (width 0.25) (layer "F.Cu") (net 4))
 (segment (start 48.325 67.2846) (end 50.1396 67.2846) (width 0.25) (layer "F.Cu") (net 4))
 (segment (start 53.275 64.7446) (end 52.0446 64.7446) (width 0.25) (layer "F.Cu") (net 9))
 (segment (start 51.562 64.262) (end 51.562 61.976) (width 0.25) (layer "F.Cu") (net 9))
 (segment (start 51.562 61.976) (end 56.34 57.198) (width 0.25) (layer "F.Cu") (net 9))
 (segment (start 56.34 57.198) (end 56.34 55.88) (width 0.25) (layer "F.Cu") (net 9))
 (segment (start 52.0446 64.7446) (end 51.562 64.262) (width 0.25) (layer "F.Cu") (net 9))
 (segment (start 50.038 61.0108) (end 52.185 58.8638) (width 0.25) (layer "F.Cu") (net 2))
 (segment (start 49.53 63.4746) (end 50.038 62.9666) (width 0.25) (layer "F.Cu") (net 2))
 (segment (start 52.185 58.8638) (end 52.185 53.04) (width 0.25) (layer "F.Cu") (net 2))
 (segment (start 48.325 63.4746) (end 49.53 63.4746) (width 0.25) (layer "F.Cu") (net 2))
 (segment (start 50.038 62.9666) (end 50.038 61.0108) (width 0.25) (layer "F.Cu") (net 2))
 (segment (start 51.054 68.0974) (end 51.054 61.6458) (width 0.25) (layer "F.Cu") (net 7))
 (segment (start 53.275 68.5546) (end 51.5112 68.5546) (width 0.25) (layer "F.Cu") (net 7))
 (segment (start 51.054 61.6458) (end 54.955 57.7448) (width 0.25) (layer "F.Cu") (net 7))
 (segment (start 51.5112 68.5546) (end 51.054 68.0974) (width 0.25) (layer "F.Cu") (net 7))
 (segment (start 54.955 57.7448) (end 54.955 53.04) (width 0.25) (layer "F.Cu") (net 7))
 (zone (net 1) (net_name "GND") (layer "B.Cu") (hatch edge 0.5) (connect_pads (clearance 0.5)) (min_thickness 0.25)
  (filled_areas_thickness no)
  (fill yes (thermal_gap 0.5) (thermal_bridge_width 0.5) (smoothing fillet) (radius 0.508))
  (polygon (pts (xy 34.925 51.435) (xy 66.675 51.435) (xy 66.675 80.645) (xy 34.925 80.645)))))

